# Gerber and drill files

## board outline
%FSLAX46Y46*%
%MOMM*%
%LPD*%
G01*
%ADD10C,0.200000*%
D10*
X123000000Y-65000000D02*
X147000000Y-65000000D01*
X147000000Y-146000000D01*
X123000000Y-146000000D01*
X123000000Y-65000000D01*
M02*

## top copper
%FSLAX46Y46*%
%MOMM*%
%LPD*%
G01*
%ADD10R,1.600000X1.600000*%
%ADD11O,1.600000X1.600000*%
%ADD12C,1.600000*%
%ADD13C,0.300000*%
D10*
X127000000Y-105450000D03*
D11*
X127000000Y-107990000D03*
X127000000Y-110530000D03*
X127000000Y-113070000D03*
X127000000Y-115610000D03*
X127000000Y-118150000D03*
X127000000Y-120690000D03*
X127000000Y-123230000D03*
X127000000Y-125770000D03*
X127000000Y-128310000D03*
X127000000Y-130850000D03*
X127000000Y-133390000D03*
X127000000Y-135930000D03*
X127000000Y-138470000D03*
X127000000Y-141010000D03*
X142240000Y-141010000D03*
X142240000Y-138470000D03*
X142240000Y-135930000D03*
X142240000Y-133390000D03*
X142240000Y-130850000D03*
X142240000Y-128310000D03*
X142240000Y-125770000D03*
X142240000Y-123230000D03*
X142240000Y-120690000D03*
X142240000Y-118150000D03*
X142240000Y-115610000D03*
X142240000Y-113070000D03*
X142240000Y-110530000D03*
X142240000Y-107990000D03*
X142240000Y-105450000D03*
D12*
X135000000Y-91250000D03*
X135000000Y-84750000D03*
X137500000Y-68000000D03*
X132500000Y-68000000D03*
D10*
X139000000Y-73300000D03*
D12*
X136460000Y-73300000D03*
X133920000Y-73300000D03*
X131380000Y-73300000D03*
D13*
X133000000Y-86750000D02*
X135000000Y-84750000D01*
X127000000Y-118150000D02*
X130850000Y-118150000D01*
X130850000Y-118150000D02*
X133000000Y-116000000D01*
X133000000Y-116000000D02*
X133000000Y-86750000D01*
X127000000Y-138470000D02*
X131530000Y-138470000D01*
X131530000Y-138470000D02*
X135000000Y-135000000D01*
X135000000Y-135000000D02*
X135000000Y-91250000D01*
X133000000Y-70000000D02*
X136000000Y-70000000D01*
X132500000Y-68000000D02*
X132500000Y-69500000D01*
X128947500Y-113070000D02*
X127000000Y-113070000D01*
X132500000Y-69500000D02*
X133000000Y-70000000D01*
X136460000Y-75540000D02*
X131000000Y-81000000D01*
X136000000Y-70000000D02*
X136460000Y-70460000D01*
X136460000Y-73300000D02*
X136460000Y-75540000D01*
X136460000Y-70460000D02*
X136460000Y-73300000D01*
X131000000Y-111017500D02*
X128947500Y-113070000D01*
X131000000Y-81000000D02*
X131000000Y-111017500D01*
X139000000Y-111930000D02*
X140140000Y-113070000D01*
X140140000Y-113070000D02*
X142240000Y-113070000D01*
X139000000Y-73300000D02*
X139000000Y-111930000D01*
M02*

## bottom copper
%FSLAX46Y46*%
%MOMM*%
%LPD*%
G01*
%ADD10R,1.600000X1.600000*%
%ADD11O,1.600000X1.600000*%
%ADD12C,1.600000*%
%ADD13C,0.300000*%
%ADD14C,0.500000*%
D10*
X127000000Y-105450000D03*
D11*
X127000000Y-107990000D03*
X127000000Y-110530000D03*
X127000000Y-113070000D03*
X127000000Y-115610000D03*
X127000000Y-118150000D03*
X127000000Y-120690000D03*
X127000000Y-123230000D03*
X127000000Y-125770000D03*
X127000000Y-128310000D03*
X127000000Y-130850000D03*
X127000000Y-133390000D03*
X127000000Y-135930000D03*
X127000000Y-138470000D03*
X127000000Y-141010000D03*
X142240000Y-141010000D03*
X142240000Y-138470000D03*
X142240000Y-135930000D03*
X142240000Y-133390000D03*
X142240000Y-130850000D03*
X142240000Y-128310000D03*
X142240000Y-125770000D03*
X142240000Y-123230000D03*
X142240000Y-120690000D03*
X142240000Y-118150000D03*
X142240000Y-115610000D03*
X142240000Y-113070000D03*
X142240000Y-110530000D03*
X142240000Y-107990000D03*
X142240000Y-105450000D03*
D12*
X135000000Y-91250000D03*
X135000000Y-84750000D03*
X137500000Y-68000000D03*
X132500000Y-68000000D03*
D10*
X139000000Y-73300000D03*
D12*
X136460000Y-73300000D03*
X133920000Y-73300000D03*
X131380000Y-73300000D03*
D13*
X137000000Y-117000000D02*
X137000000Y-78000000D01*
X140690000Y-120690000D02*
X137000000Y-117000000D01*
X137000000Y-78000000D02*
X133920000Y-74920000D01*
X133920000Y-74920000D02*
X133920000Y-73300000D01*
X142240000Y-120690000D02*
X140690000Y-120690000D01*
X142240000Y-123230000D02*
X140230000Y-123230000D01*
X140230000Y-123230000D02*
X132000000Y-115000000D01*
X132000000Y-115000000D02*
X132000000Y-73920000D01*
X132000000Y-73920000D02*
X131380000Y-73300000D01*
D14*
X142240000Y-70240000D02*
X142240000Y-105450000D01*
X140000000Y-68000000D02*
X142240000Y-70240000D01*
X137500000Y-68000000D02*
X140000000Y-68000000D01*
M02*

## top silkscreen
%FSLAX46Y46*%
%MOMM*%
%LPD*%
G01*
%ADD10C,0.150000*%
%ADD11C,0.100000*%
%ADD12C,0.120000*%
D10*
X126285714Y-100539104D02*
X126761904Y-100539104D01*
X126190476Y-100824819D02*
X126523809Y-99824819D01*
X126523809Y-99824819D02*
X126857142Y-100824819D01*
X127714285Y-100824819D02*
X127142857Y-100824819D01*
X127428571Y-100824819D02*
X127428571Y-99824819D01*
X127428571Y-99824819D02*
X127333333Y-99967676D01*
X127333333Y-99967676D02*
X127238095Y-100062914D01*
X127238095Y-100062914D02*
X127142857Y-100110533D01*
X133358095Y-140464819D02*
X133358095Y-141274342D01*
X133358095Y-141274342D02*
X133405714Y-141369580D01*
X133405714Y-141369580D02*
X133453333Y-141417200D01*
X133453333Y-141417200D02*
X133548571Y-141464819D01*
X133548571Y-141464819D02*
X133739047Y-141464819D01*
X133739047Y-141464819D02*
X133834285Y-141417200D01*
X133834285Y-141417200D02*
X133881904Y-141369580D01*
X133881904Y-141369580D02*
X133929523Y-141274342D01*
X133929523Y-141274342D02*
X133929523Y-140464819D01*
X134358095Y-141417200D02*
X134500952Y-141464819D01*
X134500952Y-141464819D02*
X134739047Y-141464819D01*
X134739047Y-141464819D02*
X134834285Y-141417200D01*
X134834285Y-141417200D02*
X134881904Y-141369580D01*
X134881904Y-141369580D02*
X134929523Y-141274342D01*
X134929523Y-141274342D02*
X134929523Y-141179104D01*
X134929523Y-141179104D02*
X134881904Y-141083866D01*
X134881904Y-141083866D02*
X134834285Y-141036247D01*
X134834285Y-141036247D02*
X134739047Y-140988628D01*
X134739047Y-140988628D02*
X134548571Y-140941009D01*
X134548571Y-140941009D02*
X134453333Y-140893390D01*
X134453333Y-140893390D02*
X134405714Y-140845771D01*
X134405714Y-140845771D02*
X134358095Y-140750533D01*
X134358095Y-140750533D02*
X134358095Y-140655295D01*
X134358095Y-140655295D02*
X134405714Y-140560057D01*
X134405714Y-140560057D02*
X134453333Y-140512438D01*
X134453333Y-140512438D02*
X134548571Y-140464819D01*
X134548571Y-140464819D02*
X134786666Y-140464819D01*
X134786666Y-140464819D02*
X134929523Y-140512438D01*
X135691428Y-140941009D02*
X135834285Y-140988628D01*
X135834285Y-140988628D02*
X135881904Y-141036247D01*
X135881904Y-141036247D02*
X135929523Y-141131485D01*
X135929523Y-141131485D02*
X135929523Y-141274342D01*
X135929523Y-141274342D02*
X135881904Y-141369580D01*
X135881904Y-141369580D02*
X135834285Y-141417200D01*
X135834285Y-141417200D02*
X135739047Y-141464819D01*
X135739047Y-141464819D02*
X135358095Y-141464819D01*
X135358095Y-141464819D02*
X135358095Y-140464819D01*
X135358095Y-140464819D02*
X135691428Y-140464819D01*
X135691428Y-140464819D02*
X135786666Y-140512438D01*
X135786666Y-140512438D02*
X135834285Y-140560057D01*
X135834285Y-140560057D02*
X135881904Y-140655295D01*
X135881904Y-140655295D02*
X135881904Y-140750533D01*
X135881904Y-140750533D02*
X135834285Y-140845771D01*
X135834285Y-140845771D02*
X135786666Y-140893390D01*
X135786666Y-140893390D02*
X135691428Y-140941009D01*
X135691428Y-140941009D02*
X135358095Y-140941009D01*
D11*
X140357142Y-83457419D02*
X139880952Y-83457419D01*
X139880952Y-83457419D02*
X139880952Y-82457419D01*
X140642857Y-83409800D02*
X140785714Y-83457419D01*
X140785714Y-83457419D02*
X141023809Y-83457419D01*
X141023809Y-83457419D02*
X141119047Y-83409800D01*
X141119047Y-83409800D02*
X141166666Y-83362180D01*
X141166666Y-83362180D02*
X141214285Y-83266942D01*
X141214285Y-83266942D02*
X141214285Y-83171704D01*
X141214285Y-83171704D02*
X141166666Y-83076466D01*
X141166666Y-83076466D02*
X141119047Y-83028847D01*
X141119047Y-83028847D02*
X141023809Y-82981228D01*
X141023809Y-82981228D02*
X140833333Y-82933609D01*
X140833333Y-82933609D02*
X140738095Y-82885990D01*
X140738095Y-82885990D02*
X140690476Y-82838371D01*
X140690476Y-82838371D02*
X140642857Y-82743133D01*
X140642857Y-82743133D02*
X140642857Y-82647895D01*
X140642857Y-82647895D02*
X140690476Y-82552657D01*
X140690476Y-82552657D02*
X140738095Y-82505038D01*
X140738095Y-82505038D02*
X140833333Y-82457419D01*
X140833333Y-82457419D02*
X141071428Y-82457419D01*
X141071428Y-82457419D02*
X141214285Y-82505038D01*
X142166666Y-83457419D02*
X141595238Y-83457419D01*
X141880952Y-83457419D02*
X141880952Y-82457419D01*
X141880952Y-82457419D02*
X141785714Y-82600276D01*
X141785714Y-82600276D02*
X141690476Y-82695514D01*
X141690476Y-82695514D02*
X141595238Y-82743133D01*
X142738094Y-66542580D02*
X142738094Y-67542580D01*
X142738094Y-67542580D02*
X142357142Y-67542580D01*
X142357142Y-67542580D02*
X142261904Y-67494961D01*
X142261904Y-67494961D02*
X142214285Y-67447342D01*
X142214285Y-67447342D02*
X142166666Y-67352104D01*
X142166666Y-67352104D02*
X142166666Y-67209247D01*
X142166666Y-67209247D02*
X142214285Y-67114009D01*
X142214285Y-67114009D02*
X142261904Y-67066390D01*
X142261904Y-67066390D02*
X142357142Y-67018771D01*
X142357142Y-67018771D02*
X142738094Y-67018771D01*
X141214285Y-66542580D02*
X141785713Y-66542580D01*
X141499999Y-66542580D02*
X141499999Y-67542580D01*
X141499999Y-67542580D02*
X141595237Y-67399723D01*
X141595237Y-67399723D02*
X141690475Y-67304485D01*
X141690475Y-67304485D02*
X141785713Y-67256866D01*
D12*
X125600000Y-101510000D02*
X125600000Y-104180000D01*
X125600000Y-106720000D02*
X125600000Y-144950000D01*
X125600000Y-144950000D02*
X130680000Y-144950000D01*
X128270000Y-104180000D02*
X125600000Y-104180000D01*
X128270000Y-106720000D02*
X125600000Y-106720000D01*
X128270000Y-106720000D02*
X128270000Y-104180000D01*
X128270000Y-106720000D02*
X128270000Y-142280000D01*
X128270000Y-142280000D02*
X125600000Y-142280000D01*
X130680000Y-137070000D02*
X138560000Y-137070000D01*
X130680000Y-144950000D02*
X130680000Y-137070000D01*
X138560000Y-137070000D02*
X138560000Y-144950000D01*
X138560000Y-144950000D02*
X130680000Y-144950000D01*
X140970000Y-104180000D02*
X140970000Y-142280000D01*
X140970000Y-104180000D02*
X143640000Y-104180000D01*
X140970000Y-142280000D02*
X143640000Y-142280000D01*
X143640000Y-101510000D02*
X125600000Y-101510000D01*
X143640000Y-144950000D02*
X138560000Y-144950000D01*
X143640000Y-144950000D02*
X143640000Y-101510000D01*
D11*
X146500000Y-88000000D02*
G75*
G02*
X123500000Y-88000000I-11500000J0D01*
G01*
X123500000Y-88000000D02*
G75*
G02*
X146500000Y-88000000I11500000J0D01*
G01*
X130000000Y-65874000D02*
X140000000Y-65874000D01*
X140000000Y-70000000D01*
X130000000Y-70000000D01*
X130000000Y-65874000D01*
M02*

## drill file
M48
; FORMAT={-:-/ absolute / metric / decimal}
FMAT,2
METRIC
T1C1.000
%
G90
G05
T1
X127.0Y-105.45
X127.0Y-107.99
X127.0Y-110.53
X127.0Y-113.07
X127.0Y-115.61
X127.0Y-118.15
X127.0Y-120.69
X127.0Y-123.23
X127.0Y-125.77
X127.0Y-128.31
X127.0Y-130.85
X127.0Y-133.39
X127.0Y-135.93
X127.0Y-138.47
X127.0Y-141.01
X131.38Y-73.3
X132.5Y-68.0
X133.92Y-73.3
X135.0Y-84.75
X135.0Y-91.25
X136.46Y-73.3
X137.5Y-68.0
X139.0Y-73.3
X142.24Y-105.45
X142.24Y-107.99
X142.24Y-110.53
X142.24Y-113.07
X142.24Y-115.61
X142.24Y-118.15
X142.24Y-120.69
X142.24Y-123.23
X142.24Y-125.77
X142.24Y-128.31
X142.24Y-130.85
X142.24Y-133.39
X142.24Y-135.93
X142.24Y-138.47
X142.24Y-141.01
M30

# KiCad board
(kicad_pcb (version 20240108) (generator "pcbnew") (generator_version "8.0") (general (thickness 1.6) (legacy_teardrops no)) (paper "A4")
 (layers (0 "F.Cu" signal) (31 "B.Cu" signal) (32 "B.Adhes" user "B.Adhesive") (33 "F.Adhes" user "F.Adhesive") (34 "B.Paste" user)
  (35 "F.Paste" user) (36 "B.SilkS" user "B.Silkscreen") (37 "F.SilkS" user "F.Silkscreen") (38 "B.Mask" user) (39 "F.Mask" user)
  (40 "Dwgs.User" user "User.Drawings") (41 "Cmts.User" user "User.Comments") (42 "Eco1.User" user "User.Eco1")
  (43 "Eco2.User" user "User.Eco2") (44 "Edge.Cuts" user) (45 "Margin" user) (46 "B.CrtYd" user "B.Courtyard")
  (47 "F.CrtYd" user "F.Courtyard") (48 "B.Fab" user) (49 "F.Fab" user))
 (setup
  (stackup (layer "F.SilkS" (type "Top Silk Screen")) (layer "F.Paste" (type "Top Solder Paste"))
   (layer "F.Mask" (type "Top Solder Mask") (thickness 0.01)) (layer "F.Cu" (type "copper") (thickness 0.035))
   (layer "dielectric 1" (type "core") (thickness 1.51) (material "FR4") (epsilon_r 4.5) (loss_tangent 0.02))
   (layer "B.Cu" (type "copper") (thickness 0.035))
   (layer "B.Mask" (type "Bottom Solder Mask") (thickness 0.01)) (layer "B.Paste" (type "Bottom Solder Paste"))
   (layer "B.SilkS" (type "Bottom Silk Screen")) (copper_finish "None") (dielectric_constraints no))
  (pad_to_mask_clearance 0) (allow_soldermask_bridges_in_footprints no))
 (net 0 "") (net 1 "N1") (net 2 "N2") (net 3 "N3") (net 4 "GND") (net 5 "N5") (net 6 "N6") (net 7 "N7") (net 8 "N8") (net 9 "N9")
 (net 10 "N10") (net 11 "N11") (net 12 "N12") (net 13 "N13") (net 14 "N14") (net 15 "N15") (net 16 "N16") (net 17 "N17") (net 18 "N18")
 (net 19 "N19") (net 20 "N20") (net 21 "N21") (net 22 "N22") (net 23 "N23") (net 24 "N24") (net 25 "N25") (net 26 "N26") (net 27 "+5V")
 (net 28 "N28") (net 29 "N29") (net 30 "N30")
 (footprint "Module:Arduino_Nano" (layer "F.Cu") (at 127 105.45)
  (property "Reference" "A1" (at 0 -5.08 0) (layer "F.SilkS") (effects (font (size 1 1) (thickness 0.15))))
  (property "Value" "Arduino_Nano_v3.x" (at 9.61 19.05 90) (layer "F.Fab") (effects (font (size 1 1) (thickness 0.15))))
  (fp_line (start -1.4 -3.94) (end -1.4 -1.27) (stroke (width 0.12) (type solid)) (layer "F.SilkS"))
  (fp_line (start -1.4 1.27) (end -1.4 39.5) (stroke (width 0.12) (type solid)) (layer "F.SilkS"))
  (fp_line (start -1.4 39.5) (end 3.68 39.5) (stroke (width 0.12) (type solid)) (layer "F.SilkS"))
  (fp_line (start 1.27 -1.27) (end -1.4 -1.27) (stroke (width 0.12) (type solid)) (layer "F.SilkS"))
  (fp_line (start 1.27 1.27) (end -1.4 1.27) (stroke (width 0.12) (type solid)) (layer "F.SilkS"))
  (fp_line (start 1.27 1.27) (end 1.27 -1.27) (stroke (width 0.12) (type solid)) (layer "F.SilkS"))
  (fp_line (start 1.27 1.27) (end 1.27 36.83) (stroke (width 0.12) (type solid)) (layer "F.SilkS"))
  (fp_line (start 1.27 36.83) (end -1.4 36.83) (stroke (width 0.12) (type solid)) (layer "F.SilkS"))
  (fp_line (start 3.68 31.62) (end 11.56 31.62) (stroke (width 0.12) (type solid)) (layer "F.SilkS"))
  (fp_line (start 3.68 39.5) (end 3.68 31.62) (stroke (width 0.12) (type solid)) (layer "F.SilkS"))
  (fp_line (start 11.56 31.62) (end 11.56 39.5) (stroke (width 0.12) (type solid)) (layer "F.SilkS"))
  (fp_line (start 11.56 39.5) (end 3.68 39.5) (stroke (width 0.12) (type solid)) (layer "F.SilkS"))
  (fp_line (start 13.97 -1.27) (end 13.97 36.83) (stroke (width 0.12) (type solid)) (layer "F.SilkS"))
  (fp_line (start 13.97 -1.27) (end 16.64 -1.27) (stroke (width 0.12) (type solid)) (layer "F.SilkS"))
  (fp_line (start 13.97 36.83) (end 16.64 36.83) (stroke (width 0.12) (type solid)) (layer "F.SilkS"))
  (fp_line (start 16.64 -3.94) (end -1.4 -3.94) (stroke (width 0.12) (type solid)) (layer "F.SilkS"))
  (fp_line (start 16.64 39.5) (end 11.56 39.5) (stroke (width 0.12) (type solid)) (layer "F.SilkS"))
  (fp_line (start 16.64 39.5) (end 16.64 -3.94) (stroke (width 0.12) (type solid)) (layer "F.SilkS"))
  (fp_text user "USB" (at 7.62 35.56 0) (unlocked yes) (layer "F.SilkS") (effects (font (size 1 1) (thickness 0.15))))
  (pad "1" thru_hole rect (at 0 0) (size 1.6 1.6) (drill 1) (layers "*.Cu" "*.Mask") (remove_unused_layers no) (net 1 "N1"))
  (pad "2" thru_hole oval (at 0 2.54) (size 1.6 1.6) (drill 1) (layers "*.Cu" "*.Mask") (remove_unused_layers no) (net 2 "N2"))
  (pad "3" thru_hole oval (at 0 5.08) (size 1.6 1.6) (drill 1) (layers "*.Cu" "*.Mask") (remove_unused_layers no) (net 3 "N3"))
  (pad "4" thru_hole oval (at 0 7.62) (size 1.6 1.6) (drill 1) (layers "*.Cu" "*.Mask") (remove_unused_layers no) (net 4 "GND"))
  (pad "5" thru_hole oval (at 0 10.16) (size 1.6 1.6) (drill 1) (layers "*.Cu" "*.Mask") (remove_unused_layers no) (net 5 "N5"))
  (pad "6" thru_hole oval (at 0 12.7) (size 1.6 1.6) (drill 1) (layers "*.Cu" "*.Mask") (remove_unused_layers no) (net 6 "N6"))
  (pad "7" thru_hole oval (at 0 15.24) (size 1.6 1.6) (drill 1) (layers "*.Cu" "*.Mask") (remove_unused_layers no) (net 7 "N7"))
  (pad "8" thru_hole oval (at 0 17.78) (size 1.6 1.6) (drill 1) (layers "*.Cu" "*.Mask") (remove_unused_layers no) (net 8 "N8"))
  (pad "9" thru_hole oval (at 0 20.32) (size 1.6 1.6) (drill 1) (layers "*.Cu" "*.Mask") (remove_unused_layers no) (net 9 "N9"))
  (pad "10" thru_hole oval (at 0 22.86) (size 1.6 1.6) (drill 1) (layers "*.Cu" "*.Mask") (remove_unused_layers no) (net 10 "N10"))
  (pad "11" thru_hole oval (at 0 25.4) (size 1.6 1.6) (drill 1) (layers "*.Cu" "*.Mask") (remove_unused_layers no) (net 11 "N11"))
  (pad "12" thru_hole oval (at 0 27.94) (size 1.6 1.6) (drill 1) (layers "*.Cu" "*.Mask") (remove_unused_layers no) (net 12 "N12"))
  (pad "13" thru_hole oval (at 0 30.48) (size 1.6 1.6) (drill 1) (layers "*.Cu" "*.Mask") (remove_unused_layers no) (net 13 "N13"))
  (pad "14" thru_hole oval (at 0 33.02) (size 1.6 1.6) (drill 1) (layers "*.Cu" "*.Mask") (remove_unused_layers no) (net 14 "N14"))
  (pad "15" thru_hole oval (at 0 35.56) (size 1.6 1.6) (drill 1) (layers "*.Cu" "*.Mask") (remove_unused_layers no) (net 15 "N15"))
  (pad "16" thru_hole oval (at 15.24 35.56) (size 1.6 1.6) (drill 1) (layers "*.Cu" "*.Mask") (remove_unused_layers no) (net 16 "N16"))
  (pad "17" thru_hole oval (at 15.24 33.02) (size 1.6 1.6) (drill 1) (layers "*.Cu" "*.Mask") (remove_unused_layers no) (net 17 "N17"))
  (pad "18" thru_hole oval (at 15.24 30.48) (size 1.6 1.6) (drill 1) (layers "*.Cu" "*.Mask") (remove_unused_layers no) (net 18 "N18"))
  (pad "19" thru_hole oval (at 15.24 27.94) (size 1.6 1.6) (drill 1) (layers "*.Cu" "*.Mask") (remove_unused_layers no) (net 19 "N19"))
  (pad "20" thru_hole oval (at 15.24 25.4) (size 1.6 1.6) (drill 1) (layers "*.Cu" "*.Mask") (remove_unused_layers no) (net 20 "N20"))
  (pad "21" thru_hole oval (at 15.24 22.86) (size 1.6 1.6) (drill 1) (layers "*.Cu" "*.Mask") (remove_unused_layers no) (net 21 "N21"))
  (pad "22" thru_hole oval (at 15.24 20.32) (size 1.6 1.6) (drill 1) (layers "*.Cu" "*.Mask") (remove_unused_layers no) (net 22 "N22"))
  (pad "23" thru_hole oval (at 15.24 17.78) (size 1.6 1.6) (drill 1) (layers "*.Cu" "*.Mask") (remove_unused_layers no) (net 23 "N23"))
  (pad "24" thru_hole oval (at 15.24 15.24) (size 1.6 1.6) (drill 1) (layers "*.Cu" "*.Mask") (remove_unused_layers no) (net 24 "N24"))
  (pad "25" thru_hole oval (at 15.24 12.7) (size 1.6 1.6) (drill 1) (layers "*.Cu" "*.Mask") (remove_unused_layers no) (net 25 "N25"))
  (pad "26" thru_hole oval (at 15.24 10.16) (size 1.6 1.6) (drill 1) (layers "*.Cu" "*.Mask") (remove_unused_layers no) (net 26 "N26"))
  (pad "27" thru_hole oval (at 15.24 7.62) (size 1.6 1.6) (drill 1) (layers "*.Cu" "*.Mask") (remove_unused_layers no) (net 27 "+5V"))
  (pad "28" thru_hole oval (at 15.24 5.08) (size 1.6 1.6) (drill 1) (layers "*.Cu" "*.Mask") (remove_unused_layers no) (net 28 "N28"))
  (pad "29" thru_hole oval (at 15.24 2.54) (size 1.6 1.6) (drill 1) (layers "*.Cu" "*.Mask") (remove_unused_layers no) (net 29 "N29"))
  (pad "30" thru_hole oval (at 15.24 0) (size 1.6 1.6) (drill 1) (layers "*.Cu" "*.Mask") (remove_unused_layers no) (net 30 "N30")))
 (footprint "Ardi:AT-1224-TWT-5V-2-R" (layer "F.Cu") (at 135 88)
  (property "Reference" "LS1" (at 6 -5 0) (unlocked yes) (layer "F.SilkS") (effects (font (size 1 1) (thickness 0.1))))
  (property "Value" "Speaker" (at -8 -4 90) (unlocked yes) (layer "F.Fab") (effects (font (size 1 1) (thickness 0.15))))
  (fp_circle (center 0 0) (end 11.5 0) (stroke (width 0.1) (type default)) (fill none) (layer "F.SilkS"))
  (pad "1" thru_hole circle (at 0 3.25) (size 1.6 1.6) (drill 1) (layers "*.Cu" "*.Mask") (remove_unused_layers no) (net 14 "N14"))
  (pad "2" thru_hole circle (at 0 -3.25) (size 1.6 1.6) (drill 1) (layers "*.Cu" "*.Mask") (remove_unused_layers no) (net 6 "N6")))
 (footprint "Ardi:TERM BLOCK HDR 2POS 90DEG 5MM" (layer "F.Cu") (at 135 64 180)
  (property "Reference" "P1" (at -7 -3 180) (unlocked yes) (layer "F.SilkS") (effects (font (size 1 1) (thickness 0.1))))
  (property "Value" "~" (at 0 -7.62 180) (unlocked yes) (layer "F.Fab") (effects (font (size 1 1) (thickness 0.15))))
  (fp_rect (start -5 -1.874) (end 5 -6) (stroke (width 0.1) (type default)) (fill none) (layer "F.SilkS"))
  (pad "1" thru_hole circle (at -2.5 -4 180) (size 1.6 1.6) (drill 1) (layers "*.Cu" "*.Mask") (remove_unused_layers no) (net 30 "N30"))
  (pad "2" thru_hole circle (at 2.5 -4 180) (size 1.6 1.6) (drill 1) (layers "*.Cu" "*.Mask") (remove_unused_layers no) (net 4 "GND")))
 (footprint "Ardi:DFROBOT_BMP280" (layer "B.Cu") (at 135.19 79.65 90)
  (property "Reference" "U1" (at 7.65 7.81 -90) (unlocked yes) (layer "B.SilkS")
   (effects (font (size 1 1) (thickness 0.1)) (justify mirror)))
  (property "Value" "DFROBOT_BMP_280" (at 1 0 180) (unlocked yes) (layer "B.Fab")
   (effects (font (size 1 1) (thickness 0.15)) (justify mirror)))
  (pad "1" thru_hole rect (at 6.35 3.81 90) (size 1.6 1.6) (drill 1) (layers "*.Cu" "*.Mask") (remove_unused_layers no) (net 27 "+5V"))
  (pad "2" thru_hole circle (at 6.35 1.27 90) (size 1.6 1.6) (drill 1) (layers "*.Cu" "*.Mask") (remove_unused_layers no) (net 4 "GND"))
  (pad "3" thru_hole circle (at 6.35 -1.27 90) (size 1.6 1.6) (drill 1) (layers "*.Cu" "*.Mask") (remove_unused_layers no) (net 24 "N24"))
  (pad "4" thru_hole circle (at 6.35 -3.81 90) (size 1.6 1.6) (drill 1) (layers "*.Cu" "*.Mask") (remove_unused_layers no) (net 23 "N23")))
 (gr_rect (start 123 65) (end 147 146) (stroke (width 0.2) (type default)) (fill none) (layer "Edge.Cuts"))
 (segment (start 133 86.75) (end 135 84.75) (width 0.3) (layer "F.Cu") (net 6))
 (segment (start 127 118.15) (end 130.85 118.15) (width 0.3) (layer "F.Cu") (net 6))
 (segment (start 130.85 118.15) (end 133 116) (width 0.3) (layer "F.Cu") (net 6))
 (segment (start 133 116) (end 133 86.75) (width 0.3) (layer "F.Cu") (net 6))
 (segment (start 127 138.47) (end 131.53 138.47) (width 0.3) (layer "F.Cu") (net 14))
 (segment (start 131.53 138.47) (end 135 135) (width 0.3) (layer "F.Cu") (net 14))
 (segment (start 135 135) (end 135 91.25) (width 0.3) (layer "F.Cu") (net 14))
 (segment (start 133 70) (end 136 70) (width 0.3) (layer "F.Cu") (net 4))
 (segment (start 132.5 68) (end 132.5 69.5) (width 0.3) (layer "F.Cu") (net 4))
 (segment (start 128.9475 113.07) (end 127 113.07) (width 0.3) (layer "F.Cu") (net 4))
 (segment (start 132.5 69.5) (end 133 70) (width 0.3) (layer "F.Cu") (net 4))
 (segment (start 136.46 75.54) (end 131 81) (width 0.3) (layer "F.Cu") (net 4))
 (segment (start 136 70) (end 136.46 70.46) (width 0.3) (layer "F.Cu") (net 4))
 (segment (start 136.46 73.3) (end 136.46 75.54) (width 0.3) (layer "F.Cu") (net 4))
 (segment (start 136.46 70.46) (end 136.46 73.3) (width 0.3) (layer "F.Cu") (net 4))
 (segment (start 131 111.0175) (end 128.9475 113.07) (width 0.3) (layer "F.Cu") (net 4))
 (segment (start 131 81) (end 131 111.0175) (width 0.3) (layer "F.Cu") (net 4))
 (segment (start 139 111.93) (end 140.14 113.07) (width 0.3) (layer "F.Cu") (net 27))
 (segment (start 140.14 113.07) (end 142.24 113.07) (width 0.3) (layer "F.Cu") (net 27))
 (segment (start 139 73.3) (end 139 111.93) (width 0.3) (layer "F.Cu") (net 27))
 (segment (start 137 117) (end 137 78) (width 0.3) (layer "B.Cu") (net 24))
 (segment (start 140.69 120.69) (end 137 117) (width 0.3) (layer "B.Cu") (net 24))
 (segment (start 137 78) (end 133.92 74.92) (width 0.3) (layer "B.Cu") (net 24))
 (segment (start 133.92 74.92) (end 133.92 73.3) (width 0.3) (layer "B.Cu") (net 24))
 (segment (start 142.24 120.69) (end 140.69 120.69) (width 0.3) (layer "B.Cu") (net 24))
 (segment (start 142.24 123.23) (end 140.23 123.23) (width 0.3) (layer "B.Cu") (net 23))
 (segment (start 140.23 123.23) (end 132 115) (width 0.3) (layer "B.Cu") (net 23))
 (segment (start 132 115) (end 132 73.92) (width 0.3) (layer "B.Cu") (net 23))
 (segment (start 132 73.92) (end 131.38 73.3) (width 0.3) (layer "B.Cu") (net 23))
 (segment (start 142.24 70.24) (end 142.24 105.45) (width 0.5) (layer "B.Cu") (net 30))
 (segment (start 140 68) (end 142.24 70.24) (width 0.5) (layer "B.Cu") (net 30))
 (segment (start 137.5 68) (end 140 68) (width 0.5) (layer "B.Cu") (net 30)))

